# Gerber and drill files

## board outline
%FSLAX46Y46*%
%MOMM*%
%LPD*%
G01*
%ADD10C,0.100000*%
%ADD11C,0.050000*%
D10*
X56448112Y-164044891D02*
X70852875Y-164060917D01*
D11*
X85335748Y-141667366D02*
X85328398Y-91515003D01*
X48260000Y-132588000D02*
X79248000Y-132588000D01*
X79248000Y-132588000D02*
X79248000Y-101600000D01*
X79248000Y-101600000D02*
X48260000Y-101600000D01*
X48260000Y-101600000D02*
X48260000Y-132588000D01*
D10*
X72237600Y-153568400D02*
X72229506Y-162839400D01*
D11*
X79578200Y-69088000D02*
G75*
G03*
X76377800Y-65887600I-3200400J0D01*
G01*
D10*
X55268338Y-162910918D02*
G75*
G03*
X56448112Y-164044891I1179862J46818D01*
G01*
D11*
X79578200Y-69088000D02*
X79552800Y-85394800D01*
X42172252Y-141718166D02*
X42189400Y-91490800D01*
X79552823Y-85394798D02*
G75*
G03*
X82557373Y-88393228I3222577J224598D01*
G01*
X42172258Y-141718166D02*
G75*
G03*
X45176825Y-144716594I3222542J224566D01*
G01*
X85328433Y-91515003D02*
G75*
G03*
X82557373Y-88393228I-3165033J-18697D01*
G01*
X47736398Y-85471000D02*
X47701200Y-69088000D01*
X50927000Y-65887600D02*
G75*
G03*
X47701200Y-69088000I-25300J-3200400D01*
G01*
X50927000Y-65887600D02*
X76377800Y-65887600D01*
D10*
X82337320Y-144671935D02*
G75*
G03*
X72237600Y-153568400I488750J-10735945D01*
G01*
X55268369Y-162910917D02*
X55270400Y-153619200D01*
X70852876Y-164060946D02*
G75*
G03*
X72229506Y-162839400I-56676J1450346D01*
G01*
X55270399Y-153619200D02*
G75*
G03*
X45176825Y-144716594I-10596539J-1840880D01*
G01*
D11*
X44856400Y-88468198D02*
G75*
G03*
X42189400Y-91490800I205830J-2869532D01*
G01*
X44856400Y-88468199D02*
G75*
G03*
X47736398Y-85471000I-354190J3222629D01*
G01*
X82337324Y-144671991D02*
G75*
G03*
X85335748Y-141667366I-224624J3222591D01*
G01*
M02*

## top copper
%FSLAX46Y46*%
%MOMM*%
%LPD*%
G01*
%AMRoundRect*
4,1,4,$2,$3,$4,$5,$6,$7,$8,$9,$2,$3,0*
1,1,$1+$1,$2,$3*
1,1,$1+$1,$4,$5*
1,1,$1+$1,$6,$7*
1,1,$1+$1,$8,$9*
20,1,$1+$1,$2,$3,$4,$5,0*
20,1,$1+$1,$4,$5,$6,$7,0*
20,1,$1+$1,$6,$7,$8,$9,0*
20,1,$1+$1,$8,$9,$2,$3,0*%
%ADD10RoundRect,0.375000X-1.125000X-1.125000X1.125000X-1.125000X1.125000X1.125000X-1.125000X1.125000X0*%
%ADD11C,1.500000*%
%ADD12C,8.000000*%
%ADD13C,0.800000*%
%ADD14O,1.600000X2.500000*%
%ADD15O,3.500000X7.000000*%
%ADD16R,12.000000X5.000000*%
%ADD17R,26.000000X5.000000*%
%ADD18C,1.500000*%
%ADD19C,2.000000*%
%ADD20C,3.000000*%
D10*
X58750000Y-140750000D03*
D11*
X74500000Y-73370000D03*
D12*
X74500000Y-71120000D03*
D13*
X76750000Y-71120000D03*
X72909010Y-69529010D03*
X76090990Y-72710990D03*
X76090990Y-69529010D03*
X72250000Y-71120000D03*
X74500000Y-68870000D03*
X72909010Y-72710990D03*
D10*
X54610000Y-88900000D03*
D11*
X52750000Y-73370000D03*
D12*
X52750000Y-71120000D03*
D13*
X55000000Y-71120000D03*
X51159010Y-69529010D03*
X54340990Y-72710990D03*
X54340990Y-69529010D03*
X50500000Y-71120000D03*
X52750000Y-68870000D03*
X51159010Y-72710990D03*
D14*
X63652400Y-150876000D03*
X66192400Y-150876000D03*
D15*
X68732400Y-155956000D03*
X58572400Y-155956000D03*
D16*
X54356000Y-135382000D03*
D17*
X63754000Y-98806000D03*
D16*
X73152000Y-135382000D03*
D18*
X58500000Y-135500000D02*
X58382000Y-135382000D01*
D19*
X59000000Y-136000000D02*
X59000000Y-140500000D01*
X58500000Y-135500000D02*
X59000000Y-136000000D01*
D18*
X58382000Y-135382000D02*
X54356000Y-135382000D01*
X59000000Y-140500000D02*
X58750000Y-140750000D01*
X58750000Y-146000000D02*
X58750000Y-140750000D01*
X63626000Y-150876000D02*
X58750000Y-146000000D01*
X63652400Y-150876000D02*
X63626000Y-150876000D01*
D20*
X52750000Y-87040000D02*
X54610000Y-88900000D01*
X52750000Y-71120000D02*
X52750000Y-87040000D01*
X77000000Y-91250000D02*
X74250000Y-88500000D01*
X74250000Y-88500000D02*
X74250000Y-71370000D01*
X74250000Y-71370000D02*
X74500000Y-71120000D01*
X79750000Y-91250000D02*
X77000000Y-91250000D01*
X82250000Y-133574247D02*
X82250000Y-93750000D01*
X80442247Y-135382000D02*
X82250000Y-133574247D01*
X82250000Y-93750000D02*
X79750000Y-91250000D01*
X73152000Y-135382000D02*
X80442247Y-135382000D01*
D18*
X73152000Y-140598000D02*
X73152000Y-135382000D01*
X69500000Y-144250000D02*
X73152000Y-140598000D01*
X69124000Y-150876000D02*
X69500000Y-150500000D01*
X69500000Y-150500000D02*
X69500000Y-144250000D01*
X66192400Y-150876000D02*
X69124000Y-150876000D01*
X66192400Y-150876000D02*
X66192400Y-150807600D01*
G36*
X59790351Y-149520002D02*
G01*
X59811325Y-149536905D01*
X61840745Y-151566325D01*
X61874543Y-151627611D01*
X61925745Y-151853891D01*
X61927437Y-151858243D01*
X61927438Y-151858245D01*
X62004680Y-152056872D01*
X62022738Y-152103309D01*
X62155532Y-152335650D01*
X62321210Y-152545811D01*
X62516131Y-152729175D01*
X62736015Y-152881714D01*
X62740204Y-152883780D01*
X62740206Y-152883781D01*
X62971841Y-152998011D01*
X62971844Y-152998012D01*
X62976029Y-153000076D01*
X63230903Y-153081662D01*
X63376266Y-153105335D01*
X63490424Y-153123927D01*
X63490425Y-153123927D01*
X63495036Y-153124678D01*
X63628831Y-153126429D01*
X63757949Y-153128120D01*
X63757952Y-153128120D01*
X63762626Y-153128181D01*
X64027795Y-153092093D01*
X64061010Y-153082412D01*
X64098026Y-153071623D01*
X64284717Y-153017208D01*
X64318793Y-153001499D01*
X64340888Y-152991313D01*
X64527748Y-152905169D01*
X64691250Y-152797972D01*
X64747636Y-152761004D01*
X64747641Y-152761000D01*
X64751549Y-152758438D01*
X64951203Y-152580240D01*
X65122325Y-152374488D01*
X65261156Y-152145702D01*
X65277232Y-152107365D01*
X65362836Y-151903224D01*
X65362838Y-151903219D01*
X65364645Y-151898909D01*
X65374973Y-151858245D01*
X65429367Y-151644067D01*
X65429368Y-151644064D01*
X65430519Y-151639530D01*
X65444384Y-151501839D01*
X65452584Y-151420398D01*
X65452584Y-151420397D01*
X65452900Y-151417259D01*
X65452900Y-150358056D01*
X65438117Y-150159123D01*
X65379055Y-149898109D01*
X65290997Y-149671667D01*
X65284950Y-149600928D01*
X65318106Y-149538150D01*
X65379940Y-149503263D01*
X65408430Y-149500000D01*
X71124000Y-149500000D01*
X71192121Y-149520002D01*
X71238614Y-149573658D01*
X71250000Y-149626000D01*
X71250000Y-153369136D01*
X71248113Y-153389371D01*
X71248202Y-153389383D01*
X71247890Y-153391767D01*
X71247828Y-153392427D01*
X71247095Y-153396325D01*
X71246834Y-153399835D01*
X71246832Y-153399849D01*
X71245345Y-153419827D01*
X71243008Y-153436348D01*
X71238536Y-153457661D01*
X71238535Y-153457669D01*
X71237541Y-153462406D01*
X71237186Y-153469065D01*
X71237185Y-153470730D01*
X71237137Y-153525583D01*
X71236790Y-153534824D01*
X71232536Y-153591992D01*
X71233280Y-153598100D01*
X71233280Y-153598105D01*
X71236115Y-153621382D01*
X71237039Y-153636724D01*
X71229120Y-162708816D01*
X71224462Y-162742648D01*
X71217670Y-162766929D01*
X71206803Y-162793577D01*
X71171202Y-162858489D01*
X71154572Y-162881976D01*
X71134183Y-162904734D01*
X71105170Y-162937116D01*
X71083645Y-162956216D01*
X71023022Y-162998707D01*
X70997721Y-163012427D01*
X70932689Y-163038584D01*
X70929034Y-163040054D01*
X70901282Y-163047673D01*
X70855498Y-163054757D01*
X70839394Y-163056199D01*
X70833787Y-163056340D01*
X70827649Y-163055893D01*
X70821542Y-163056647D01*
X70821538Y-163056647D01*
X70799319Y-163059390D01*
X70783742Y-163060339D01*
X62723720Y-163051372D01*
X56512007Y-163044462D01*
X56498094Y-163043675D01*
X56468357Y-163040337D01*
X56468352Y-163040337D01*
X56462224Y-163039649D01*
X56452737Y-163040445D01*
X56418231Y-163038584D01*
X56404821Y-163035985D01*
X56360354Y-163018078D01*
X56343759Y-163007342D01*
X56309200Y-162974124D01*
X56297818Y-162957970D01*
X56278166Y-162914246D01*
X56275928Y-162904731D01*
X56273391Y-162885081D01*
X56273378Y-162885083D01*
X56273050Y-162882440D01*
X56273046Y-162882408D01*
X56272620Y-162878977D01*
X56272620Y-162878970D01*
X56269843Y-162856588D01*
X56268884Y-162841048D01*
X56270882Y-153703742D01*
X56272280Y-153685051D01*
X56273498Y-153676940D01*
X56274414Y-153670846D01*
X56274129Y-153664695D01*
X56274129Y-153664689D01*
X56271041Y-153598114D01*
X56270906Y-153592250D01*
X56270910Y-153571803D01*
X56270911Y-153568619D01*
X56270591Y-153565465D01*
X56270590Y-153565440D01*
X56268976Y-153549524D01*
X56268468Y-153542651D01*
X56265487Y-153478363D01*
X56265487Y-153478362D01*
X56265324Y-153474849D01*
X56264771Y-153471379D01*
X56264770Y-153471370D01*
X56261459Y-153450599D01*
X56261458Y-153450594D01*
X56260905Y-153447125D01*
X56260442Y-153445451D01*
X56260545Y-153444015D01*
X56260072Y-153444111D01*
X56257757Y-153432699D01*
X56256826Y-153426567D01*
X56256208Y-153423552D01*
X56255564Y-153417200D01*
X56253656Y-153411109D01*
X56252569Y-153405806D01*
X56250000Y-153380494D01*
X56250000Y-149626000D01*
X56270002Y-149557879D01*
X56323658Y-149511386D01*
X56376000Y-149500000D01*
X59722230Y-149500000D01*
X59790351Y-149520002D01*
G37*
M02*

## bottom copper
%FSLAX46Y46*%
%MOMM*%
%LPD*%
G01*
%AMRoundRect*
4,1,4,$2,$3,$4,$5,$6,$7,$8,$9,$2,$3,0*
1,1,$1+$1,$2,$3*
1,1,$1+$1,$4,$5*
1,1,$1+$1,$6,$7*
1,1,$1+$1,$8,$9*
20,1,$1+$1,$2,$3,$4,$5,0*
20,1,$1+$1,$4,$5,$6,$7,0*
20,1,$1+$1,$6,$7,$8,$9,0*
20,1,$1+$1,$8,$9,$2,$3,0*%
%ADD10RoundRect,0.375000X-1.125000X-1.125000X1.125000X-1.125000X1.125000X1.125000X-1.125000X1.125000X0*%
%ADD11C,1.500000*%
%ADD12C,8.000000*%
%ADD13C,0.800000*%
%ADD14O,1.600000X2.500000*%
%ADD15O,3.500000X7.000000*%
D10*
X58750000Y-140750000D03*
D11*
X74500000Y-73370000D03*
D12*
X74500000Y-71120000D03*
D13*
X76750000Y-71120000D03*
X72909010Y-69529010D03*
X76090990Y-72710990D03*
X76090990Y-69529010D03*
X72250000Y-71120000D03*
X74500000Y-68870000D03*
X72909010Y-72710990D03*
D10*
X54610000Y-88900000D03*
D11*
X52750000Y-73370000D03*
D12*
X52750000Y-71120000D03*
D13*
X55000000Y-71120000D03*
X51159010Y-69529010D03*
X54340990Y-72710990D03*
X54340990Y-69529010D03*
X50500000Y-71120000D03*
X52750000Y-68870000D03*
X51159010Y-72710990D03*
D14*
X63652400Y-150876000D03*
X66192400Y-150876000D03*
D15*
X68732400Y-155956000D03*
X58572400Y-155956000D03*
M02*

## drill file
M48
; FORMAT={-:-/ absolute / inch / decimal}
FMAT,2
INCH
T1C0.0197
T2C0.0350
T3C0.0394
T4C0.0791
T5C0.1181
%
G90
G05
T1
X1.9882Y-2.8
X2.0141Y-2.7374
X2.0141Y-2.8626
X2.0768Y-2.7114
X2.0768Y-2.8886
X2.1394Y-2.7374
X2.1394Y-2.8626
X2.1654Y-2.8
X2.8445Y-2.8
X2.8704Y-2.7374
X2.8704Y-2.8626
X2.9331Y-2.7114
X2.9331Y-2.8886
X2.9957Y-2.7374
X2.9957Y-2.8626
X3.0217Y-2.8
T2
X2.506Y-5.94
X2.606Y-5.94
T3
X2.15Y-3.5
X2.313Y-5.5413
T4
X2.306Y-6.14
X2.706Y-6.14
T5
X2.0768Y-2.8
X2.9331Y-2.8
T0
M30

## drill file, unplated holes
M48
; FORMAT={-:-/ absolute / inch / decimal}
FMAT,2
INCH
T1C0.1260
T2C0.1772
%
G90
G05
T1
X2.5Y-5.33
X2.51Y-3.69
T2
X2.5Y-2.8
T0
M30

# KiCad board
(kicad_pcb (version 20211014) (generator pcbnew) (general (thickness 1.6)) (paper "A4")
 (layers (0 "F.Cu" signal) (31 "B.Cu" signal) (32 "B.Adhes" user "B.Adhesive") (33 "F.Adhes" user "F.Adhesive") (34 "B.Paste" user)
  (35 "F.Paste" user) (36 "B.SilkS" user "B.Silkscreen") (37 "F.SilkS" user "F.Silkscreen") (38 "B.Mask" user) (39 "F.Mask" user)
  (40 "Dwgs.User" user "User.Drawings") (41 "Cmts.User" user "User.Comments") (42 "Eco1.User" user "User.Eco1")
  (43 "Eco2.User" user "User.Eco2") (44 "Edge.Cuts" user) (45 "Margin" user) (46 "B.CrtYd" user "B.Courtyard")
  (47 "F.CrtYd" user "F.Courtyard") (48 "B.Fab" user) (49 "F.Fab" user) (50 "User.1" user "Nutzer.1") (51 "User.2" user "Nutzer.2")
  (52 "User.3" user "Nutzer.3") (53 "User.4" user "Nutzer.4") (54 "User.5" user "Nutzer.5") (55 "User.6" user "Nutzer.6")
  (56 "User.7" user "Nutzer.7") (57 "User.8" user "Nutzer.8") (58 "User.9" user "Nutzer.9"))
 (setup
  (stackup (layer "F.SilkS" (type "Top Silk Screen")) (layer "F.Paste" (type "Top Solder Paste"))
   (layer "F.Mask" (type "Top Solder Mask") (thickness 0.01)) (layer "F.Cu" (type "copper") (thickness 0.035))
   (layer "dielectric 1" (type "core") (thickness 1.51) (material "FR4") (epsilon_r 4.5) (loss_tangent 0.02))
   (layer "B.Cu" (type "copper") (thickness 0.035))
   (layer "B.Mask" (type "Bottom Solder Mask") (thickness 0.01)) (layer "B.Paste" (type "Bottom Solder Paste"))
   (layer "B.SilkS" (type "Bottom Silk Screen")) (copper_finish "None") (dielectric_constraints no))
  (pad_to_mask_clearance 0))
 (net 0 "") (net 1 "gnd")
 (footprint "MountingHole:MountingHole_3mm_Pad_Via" (layer "F.Cu") (at 74.5 71.12)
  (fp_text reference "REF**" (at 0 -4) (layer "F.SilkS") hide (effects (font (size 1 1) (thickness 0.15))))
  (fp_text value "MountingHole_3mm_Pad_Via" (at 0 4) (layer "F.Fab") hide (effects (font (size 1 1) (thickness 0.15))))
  (pad "1" thru_hole circle (at 0 2.25) (size 1.5 1.5) (drill 0.5) (layers *.Cu *.Mask) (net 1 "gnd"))
  (pad "1" thru_hole circle (at 0 0) (size 8 8) (drill 3) (layers *.Cu *.Mask) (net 1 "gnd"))
  (pad "1" thru_hole circle (at 2.25 0) (size 0.8 0.8) (drill 0.5) (layers *.Cu *.Mask) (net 1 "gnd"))
  (pad "1" thru_hole circle (at -1.59099 -1.59099) (size 0.8 0.8) (drill 0.5) (layers *.Cu *.Mask) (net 1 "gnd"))
  (pad "1" thru_hole circle (at 1.59099 1.59099) (size 0.8 0.8) (drill 0.5) (layers *.Cu *.Mask) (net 1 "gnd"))
  (pad "1" thru_hole circle (at 1.59099 -1.59099) (size 0.8 0.8) (drill 0.5) (layers *.Cu *.Mask) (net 1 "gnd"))
  (pad "1" thru_hole circle (at -2.25 0) (size 0.8 0.8) (drill 0.5) (layers *.Cu *.Mask) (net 1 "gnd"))
  (pad "1" thru_hole circle (at 0 -2.25) (size 0.8 0.8) (drill 0.5) (layers *.Cu *.Mask) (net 1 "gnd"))
  (pad "1" thru_hole circle (at -1.59099 1.59099) (size 0.8 0.8) (drill 0.5) (layers *.Cu *.Mask) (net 1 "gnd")))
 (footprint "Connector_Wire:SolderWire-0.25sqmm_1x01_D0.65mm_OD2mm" (layer "F.Cu") (at 54.61 88.9)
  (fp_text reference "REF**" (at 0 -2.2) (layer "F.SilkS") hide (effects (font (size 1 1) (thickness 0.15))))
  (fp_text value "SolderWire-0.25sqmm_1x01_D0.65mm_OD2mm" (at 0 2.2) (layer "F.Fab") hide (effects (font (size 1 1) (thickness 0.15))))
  (pad "1" thru_hole roundrect (at 0 0) (size 3 3) (drill 1) (layers *.Cu *.Mask) (roundrect_rratio 0.125)))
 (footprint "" (layer "F.Cu") (at 63.754 93.726)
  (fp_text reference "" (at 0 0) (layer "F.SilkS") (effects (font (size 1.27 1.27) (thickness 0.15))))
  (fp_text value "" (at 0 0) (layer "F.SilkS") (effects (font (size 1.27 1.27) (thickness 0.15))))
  (pad "" np_thru_hole circle (at 0 0) (size 3.2 3.2) (drill 3.2) (layers *.Cu *.Mask)))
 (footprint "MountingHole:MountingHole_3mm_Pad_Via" (layer "F.Cu") (at 52.75 71.12)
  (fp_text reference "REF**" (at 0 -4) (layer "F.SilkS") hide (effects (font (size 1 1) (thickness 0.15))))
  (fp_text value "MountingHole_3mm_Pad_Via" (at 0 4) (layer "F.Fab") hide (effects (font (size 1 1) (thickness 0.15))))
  (pad "1" thru_hole circle (at 1.59099 -1.59099) (size 0.8 0.8) (drill 0.5) (layers *.Cu *.Mask))
  (pad "1" thru_hole circle (at 1.59099 1.59099) (size 0.8 0.8) (drill 0.5) (layers *.Cu *.Mask))
  (pad "1" thru_hole circle (at 0 0) (size 8 8) (drill 3) (layers *.Cu *.Mask))
  (pad "1" thru_hole circle (at -1.59099 -1.59099) (size 0.8 0.8) (drill 0.5) (layers *.Cu *.Mask))
  (pad "1" thru_hole circle (at 0 -2.25) (size 0.8 0.8) (drill 0.5) (layers *.Cu *.Mask))
  (pad "1" thru_hole circle (at -2.25 0) (size 0.8 0.8) (drill 0.5) (layers *.Cu *.Mask))
  (pad "1" thru_hole circle (at 0 2.25) (size 1.5 1.5) (drill 0.5) (layers *.Cu *.Mask))
  (pad "1" thru_hole circle (at -1.59099 1.59099) (size 0.8 0.8) (drill 0.5) (layers *.Cu *.Mask))
  (pad "1" thru_hole circle (at 2.25 0) (size 0.8 0.8) (drill 0.5) (layers *.Cu *.Mask)))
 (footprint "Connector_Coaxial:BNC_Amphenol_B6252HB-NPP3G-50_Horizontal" (layer "F.Cu") (at 63.6524 150.876 180)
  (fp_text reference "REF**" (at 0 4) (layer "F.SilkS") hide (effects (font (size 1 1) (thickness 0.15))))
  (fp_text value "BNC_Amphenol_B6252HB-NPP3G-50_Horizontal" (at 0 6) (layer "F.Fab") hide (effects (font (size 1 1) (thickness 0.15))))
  (pad "1" thru_hole oval (at 0 0 180) (size 1.6 2.5) (drill 0.89) (layers *.Cu *.Mask))
  (pad "2" thru_hole oval (at -2.54 0 180) (size 1.6 2.5) (drill 0.89) (layers *.Cu *.Mask) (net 1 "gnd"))
  (pad "2" thru_hole oval (at -5.08 -5.08 180) (size 3.5 7) (drill 2.01) (layers *.Cu *.Mask) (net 1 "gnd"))
  (pad "2" thru_hole oval (at 5.08 -5.08 180) (size 3.5 7) (drill 2.01) (layers *.Cu *.Mask) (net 1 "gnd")))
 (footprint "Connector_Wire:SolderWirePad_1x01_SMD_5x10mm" (layer "F.Cu") (at 54.356 135.382 90)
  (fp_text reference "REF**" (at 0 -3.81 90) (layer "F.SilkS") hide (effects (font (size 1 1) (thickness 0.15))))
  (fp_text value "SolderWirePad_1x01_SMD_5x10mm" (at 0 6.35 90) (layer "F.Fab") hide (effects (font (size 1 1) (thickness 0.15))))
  (pad "1" smd rect (at 0 0 90) (size 5 12) (layers "F.Cu" "F.Paste" "F.Mask")))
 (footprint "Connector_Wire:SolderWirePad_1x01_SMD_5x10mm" (layer "F.Cu") (at 63.754 98.806 90)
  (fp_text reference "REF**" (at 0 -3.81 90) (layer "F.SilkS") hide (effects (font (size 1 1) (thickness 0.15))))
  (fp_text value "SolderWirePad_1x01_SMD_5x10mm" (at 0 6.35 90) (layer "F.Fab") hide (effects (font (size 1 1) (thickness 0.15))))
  (pad "1" smd rect (at 0 0 90) (size 5 26) (layers "F.Cu" "F.Paste" "F.Mask")))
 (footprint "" (layer "F.Cu") (at 73.152 135.382)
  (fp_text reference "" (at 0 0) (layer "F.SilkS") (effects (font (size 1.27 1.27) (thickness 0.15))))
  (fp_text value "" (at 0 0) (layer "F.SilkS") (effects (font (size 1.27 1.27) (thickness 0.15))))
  (pad "1" smd rect (at 0 0 90) (size 5 12) (layers "F.Cu" "F.Paste" "F.Mask") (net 1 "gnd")))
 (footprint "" (layer "F.Cu") (at 58.75 140.75)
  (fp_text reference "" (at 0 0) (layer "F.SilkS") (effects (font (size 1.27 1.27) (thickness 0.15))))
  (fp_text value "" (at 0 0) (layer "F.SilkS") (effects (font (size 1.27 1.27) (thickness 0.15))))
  (pad "1" thru_hole roundrect (at 0 0) (size 3 3) (drill 1) (layers *.Cu *.Mask) (roundrect_rratio 0.125)))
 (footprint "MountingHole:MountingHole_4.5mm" (layer "F.Cu") (at 63.5 71.12)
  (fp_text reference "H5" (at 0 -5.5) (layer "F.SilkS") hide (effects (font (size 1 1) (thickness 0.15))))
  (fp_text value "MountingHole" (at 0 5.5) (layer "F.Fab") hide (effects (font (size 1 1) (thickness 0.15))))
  (pad "" np_thru_hole circle (at 0 0) (size 4.5 4.5) (drill 4.5) (layers *.Cu *.Mask)))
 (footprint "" (layer "F.Cu") (at 63.5 135.382)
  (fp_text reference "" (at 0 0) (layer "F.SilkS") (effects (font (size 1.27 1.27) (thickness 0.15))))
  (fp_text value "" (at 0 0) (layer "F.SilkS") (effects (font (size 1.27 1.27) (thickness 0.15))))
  (pad "" np_thru_hole circle (at 0 0) (size 3.2 3.2) (drill 3.2) (layers *.Cu *.Mask)))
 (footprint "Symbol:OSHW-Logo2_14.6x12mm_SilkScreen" (layer "B.Cu") (at 63.75 94.5 180)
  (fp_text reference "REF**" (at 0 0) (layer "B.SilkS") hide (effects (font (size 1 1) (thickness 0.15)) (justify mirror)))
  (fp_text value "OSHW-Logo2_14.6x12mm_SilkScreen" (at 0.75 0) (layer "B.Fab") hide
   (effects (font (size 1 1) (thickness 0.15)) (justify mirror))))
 (gr_line (start 56.448112 164.044891) (end 70.852875 164.060917) (layer "Edge.Cuts") (width 0.1))
 (gr_line (start 85.335748 141.667366) (end 85.328398 91.515003) (layer "Edge.Cuts") (width 0.05))
 (gr_rect (start 48.26 132.588) (end 79.248 101.6) (layer "Edge.Cuts") (width 0.05) (fill none))
 (gr_line (start 72.2376 153.5684) (end 72.229506 162.8394) (layer "Edge.Cuts") (width 0.1))
 (gr_arc (start 76.3778 65.8876) (mid 78.640825 66.824975) (end 79.5782 69.088) (layer "Edge.Cuts") (width 0.05))
 (gr_arc (start 56.448112 164.044891) (mid 55.629956 163.715403) (end 55.268369 162.910917) (layer "Edge.Cuts") (width 0.1))
 (gr_line (start 79.5782 69.088) (end 79.5528 85.3948) (layer "Edge.Cuts") (width 0.05))
 (gr_line (start 42.172252 141.718166) (end 42.1894 91.4908) (layer "Edge.Cuts") (width 0.05))
 (gr_arc (start 82.557373 88.393228) (mid 80.493484 87.456768) (end 79.5528 85.3948) (layer "Edge.Cuts") (width 0.05))
 (gr_arc (start 45.176825 144.716594) (mid 43.112934 143.780135) (end 42.172252 141.718166) (layer "Edge.Cuts") (width 0.05))
 (gr_arc (start 82.557373 88.393228) (mid 84.5312 89.4334) (end 85.328398 91.515003) (layer "Edge.Cuts") (width 0.05))
 (gr_line (start 47.736398 85.471) (end 47.7012 69.088) (layer "Edge.Cuts") (width 0.05))
 (gr_arc (start 47.7012 69.088) (mid 48.647567 66.815977) (end 50.927 65.8876) (layer "Edge.Cuts") (width 0.05))
 (gr_line (start 50.927 65.8876) (end 76.3778 65.8876) (layer "Edge.Cuts") (width 0.05))
 (gr_arc (start 72.2376 153.5684) (mid 75.722341 147.343366) (end 82.33732 144.671939) (layer "Edge.Cuts") (width 0.1))
 (gr_line (start 55.268369 162.910917) (end 55.2704 153.6192) (layer "Edge.Cuts") (width 0.1))
 (gr_arc (start 72.229506 162.8394) (mid 71.759551 163.696247) (end 70.852875 164.060917) (layer "Edge.Cuts") (width 0.1))
 (gr_arc (start 45.176825 144.716594) (mid 51.788201 147.394001) (end 55.2704 153.6192) (layer "Edge.Cuts") (width 0.1))
 (gr_arc (start 42.1894 91.4908) (mid 42.908353 89.430537) (end 44.8564 88.4682) (layer "Edge.Cuts") (width 0.05))
 (gr_arc (start 47.736398 85.471) (mid 46.839926 87.491873) (end 44.8564 88.4682) (layer "Edge.Cuts") (width 0.05))
 (gr_arc (start 85.335748 141.667366) (mid 84.399289 143.731257) (end 82.33732 144.671939) (layer "Edge.Cuts") (width 0.05))
 (segment (start 63.626 150.876) (end 58.75 146) (width 1.5) (layer "F.Cu") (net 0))
 (segment (start 58.5 135.5) (end 58.382 135.382) (width 1.5) (layer "F.Cu") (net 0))
 (segment (start 52.75 71.12) (end 52.75 87.04) (width 3) (layer "F.Cu") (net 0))
 (segment (start 58.5 135.5) (end 59 136) (width 2) (layer "F.Cu") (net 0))
 (segment (start 52.75 87.04) (end 54.61 88.9) (width 3) (layer "F.Cu") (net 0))
 (segment (start 59 136) (end 59 140.5) (width 2) (layer "F.Cu") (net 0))
 (segment (start 63.6524 150.876) (end 63.626 150.876) (width 1.5) (layer "F.Cu") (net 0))
 (segment (start 58.75 146) (end 58.75 140.75) (width 1.5) (layer "F.Cu") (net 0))
 (segment (start 59 140.5) (end 58.75 140.75) (width 1.5) (layer "F.Cu") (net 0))
 (segment (start 58.382 135.382) (end 54.356 135.382) (width 1.5) (layer "F.Cu") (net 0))
 (segment (start 73.152 140.598) (end 73.152 135.382) (width 1.5) (layer "F.Cu") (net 1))
 (segment (start 80.442247 135.382) (end 82.25 133.574247) (width 3) (layer "F.Cu") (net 1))
 (segment (start 82.25 93.75) (end 79.75 91.25) (width 3) (layer "F.Cu") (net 1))
 (segment (start 69.5 144.25) (end 73.152 140.598) (width 1.5) (layer "F.Cu") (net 1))
 (segment (start 77 91.25) (end 74.25 88.5) (width 3) (layer "F.Cu") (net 1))
 (segment (start 74.25 71.37) (end 74.5 71.12) (width 3) (layer "F.Cu") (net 1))
 (segment (start 82.25 133.574247) (end 82.25 93.75) (width 3) (layer "F.Cu") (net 1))
 (segment (start 74.25 88.5) (end 74.25 71.37) (width 3) (layer "F.Cu") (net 1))
 (segment (start 69.124 150.876) (end 69.5 150.5) (width 1.5) (layer "F.Cu") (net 1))
 (segment (start 69.5 150.5) (end 69.5 144.25) (width 1.5) (layer "F.Cu") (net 1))
 (segment (start 73.152 135.382) (end 80.442247 135.382) (width 3) (layer "F.Cu") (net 1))
 (segment (start 66.1924 150.876) (end 69.124 150.876) (width 1.5) (layer "F.Cu") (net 1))
 (segment (start 79.75 91.25) (end 77 91.25) (width 3) (layer "F.Cu") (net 1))
 (segment (start 66.1924 150.876) (end 66.1924 150.8076) (width 1.5) (layer "F.Cu") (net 1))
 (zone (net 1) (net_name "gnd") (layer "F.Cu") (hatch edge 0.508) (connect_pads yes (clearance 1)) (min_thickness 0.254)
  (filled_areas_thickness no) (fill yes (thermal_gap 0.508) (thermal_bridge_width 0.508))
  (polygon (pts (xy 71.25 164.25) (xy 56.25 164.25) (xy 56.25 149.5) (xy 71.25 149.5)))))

